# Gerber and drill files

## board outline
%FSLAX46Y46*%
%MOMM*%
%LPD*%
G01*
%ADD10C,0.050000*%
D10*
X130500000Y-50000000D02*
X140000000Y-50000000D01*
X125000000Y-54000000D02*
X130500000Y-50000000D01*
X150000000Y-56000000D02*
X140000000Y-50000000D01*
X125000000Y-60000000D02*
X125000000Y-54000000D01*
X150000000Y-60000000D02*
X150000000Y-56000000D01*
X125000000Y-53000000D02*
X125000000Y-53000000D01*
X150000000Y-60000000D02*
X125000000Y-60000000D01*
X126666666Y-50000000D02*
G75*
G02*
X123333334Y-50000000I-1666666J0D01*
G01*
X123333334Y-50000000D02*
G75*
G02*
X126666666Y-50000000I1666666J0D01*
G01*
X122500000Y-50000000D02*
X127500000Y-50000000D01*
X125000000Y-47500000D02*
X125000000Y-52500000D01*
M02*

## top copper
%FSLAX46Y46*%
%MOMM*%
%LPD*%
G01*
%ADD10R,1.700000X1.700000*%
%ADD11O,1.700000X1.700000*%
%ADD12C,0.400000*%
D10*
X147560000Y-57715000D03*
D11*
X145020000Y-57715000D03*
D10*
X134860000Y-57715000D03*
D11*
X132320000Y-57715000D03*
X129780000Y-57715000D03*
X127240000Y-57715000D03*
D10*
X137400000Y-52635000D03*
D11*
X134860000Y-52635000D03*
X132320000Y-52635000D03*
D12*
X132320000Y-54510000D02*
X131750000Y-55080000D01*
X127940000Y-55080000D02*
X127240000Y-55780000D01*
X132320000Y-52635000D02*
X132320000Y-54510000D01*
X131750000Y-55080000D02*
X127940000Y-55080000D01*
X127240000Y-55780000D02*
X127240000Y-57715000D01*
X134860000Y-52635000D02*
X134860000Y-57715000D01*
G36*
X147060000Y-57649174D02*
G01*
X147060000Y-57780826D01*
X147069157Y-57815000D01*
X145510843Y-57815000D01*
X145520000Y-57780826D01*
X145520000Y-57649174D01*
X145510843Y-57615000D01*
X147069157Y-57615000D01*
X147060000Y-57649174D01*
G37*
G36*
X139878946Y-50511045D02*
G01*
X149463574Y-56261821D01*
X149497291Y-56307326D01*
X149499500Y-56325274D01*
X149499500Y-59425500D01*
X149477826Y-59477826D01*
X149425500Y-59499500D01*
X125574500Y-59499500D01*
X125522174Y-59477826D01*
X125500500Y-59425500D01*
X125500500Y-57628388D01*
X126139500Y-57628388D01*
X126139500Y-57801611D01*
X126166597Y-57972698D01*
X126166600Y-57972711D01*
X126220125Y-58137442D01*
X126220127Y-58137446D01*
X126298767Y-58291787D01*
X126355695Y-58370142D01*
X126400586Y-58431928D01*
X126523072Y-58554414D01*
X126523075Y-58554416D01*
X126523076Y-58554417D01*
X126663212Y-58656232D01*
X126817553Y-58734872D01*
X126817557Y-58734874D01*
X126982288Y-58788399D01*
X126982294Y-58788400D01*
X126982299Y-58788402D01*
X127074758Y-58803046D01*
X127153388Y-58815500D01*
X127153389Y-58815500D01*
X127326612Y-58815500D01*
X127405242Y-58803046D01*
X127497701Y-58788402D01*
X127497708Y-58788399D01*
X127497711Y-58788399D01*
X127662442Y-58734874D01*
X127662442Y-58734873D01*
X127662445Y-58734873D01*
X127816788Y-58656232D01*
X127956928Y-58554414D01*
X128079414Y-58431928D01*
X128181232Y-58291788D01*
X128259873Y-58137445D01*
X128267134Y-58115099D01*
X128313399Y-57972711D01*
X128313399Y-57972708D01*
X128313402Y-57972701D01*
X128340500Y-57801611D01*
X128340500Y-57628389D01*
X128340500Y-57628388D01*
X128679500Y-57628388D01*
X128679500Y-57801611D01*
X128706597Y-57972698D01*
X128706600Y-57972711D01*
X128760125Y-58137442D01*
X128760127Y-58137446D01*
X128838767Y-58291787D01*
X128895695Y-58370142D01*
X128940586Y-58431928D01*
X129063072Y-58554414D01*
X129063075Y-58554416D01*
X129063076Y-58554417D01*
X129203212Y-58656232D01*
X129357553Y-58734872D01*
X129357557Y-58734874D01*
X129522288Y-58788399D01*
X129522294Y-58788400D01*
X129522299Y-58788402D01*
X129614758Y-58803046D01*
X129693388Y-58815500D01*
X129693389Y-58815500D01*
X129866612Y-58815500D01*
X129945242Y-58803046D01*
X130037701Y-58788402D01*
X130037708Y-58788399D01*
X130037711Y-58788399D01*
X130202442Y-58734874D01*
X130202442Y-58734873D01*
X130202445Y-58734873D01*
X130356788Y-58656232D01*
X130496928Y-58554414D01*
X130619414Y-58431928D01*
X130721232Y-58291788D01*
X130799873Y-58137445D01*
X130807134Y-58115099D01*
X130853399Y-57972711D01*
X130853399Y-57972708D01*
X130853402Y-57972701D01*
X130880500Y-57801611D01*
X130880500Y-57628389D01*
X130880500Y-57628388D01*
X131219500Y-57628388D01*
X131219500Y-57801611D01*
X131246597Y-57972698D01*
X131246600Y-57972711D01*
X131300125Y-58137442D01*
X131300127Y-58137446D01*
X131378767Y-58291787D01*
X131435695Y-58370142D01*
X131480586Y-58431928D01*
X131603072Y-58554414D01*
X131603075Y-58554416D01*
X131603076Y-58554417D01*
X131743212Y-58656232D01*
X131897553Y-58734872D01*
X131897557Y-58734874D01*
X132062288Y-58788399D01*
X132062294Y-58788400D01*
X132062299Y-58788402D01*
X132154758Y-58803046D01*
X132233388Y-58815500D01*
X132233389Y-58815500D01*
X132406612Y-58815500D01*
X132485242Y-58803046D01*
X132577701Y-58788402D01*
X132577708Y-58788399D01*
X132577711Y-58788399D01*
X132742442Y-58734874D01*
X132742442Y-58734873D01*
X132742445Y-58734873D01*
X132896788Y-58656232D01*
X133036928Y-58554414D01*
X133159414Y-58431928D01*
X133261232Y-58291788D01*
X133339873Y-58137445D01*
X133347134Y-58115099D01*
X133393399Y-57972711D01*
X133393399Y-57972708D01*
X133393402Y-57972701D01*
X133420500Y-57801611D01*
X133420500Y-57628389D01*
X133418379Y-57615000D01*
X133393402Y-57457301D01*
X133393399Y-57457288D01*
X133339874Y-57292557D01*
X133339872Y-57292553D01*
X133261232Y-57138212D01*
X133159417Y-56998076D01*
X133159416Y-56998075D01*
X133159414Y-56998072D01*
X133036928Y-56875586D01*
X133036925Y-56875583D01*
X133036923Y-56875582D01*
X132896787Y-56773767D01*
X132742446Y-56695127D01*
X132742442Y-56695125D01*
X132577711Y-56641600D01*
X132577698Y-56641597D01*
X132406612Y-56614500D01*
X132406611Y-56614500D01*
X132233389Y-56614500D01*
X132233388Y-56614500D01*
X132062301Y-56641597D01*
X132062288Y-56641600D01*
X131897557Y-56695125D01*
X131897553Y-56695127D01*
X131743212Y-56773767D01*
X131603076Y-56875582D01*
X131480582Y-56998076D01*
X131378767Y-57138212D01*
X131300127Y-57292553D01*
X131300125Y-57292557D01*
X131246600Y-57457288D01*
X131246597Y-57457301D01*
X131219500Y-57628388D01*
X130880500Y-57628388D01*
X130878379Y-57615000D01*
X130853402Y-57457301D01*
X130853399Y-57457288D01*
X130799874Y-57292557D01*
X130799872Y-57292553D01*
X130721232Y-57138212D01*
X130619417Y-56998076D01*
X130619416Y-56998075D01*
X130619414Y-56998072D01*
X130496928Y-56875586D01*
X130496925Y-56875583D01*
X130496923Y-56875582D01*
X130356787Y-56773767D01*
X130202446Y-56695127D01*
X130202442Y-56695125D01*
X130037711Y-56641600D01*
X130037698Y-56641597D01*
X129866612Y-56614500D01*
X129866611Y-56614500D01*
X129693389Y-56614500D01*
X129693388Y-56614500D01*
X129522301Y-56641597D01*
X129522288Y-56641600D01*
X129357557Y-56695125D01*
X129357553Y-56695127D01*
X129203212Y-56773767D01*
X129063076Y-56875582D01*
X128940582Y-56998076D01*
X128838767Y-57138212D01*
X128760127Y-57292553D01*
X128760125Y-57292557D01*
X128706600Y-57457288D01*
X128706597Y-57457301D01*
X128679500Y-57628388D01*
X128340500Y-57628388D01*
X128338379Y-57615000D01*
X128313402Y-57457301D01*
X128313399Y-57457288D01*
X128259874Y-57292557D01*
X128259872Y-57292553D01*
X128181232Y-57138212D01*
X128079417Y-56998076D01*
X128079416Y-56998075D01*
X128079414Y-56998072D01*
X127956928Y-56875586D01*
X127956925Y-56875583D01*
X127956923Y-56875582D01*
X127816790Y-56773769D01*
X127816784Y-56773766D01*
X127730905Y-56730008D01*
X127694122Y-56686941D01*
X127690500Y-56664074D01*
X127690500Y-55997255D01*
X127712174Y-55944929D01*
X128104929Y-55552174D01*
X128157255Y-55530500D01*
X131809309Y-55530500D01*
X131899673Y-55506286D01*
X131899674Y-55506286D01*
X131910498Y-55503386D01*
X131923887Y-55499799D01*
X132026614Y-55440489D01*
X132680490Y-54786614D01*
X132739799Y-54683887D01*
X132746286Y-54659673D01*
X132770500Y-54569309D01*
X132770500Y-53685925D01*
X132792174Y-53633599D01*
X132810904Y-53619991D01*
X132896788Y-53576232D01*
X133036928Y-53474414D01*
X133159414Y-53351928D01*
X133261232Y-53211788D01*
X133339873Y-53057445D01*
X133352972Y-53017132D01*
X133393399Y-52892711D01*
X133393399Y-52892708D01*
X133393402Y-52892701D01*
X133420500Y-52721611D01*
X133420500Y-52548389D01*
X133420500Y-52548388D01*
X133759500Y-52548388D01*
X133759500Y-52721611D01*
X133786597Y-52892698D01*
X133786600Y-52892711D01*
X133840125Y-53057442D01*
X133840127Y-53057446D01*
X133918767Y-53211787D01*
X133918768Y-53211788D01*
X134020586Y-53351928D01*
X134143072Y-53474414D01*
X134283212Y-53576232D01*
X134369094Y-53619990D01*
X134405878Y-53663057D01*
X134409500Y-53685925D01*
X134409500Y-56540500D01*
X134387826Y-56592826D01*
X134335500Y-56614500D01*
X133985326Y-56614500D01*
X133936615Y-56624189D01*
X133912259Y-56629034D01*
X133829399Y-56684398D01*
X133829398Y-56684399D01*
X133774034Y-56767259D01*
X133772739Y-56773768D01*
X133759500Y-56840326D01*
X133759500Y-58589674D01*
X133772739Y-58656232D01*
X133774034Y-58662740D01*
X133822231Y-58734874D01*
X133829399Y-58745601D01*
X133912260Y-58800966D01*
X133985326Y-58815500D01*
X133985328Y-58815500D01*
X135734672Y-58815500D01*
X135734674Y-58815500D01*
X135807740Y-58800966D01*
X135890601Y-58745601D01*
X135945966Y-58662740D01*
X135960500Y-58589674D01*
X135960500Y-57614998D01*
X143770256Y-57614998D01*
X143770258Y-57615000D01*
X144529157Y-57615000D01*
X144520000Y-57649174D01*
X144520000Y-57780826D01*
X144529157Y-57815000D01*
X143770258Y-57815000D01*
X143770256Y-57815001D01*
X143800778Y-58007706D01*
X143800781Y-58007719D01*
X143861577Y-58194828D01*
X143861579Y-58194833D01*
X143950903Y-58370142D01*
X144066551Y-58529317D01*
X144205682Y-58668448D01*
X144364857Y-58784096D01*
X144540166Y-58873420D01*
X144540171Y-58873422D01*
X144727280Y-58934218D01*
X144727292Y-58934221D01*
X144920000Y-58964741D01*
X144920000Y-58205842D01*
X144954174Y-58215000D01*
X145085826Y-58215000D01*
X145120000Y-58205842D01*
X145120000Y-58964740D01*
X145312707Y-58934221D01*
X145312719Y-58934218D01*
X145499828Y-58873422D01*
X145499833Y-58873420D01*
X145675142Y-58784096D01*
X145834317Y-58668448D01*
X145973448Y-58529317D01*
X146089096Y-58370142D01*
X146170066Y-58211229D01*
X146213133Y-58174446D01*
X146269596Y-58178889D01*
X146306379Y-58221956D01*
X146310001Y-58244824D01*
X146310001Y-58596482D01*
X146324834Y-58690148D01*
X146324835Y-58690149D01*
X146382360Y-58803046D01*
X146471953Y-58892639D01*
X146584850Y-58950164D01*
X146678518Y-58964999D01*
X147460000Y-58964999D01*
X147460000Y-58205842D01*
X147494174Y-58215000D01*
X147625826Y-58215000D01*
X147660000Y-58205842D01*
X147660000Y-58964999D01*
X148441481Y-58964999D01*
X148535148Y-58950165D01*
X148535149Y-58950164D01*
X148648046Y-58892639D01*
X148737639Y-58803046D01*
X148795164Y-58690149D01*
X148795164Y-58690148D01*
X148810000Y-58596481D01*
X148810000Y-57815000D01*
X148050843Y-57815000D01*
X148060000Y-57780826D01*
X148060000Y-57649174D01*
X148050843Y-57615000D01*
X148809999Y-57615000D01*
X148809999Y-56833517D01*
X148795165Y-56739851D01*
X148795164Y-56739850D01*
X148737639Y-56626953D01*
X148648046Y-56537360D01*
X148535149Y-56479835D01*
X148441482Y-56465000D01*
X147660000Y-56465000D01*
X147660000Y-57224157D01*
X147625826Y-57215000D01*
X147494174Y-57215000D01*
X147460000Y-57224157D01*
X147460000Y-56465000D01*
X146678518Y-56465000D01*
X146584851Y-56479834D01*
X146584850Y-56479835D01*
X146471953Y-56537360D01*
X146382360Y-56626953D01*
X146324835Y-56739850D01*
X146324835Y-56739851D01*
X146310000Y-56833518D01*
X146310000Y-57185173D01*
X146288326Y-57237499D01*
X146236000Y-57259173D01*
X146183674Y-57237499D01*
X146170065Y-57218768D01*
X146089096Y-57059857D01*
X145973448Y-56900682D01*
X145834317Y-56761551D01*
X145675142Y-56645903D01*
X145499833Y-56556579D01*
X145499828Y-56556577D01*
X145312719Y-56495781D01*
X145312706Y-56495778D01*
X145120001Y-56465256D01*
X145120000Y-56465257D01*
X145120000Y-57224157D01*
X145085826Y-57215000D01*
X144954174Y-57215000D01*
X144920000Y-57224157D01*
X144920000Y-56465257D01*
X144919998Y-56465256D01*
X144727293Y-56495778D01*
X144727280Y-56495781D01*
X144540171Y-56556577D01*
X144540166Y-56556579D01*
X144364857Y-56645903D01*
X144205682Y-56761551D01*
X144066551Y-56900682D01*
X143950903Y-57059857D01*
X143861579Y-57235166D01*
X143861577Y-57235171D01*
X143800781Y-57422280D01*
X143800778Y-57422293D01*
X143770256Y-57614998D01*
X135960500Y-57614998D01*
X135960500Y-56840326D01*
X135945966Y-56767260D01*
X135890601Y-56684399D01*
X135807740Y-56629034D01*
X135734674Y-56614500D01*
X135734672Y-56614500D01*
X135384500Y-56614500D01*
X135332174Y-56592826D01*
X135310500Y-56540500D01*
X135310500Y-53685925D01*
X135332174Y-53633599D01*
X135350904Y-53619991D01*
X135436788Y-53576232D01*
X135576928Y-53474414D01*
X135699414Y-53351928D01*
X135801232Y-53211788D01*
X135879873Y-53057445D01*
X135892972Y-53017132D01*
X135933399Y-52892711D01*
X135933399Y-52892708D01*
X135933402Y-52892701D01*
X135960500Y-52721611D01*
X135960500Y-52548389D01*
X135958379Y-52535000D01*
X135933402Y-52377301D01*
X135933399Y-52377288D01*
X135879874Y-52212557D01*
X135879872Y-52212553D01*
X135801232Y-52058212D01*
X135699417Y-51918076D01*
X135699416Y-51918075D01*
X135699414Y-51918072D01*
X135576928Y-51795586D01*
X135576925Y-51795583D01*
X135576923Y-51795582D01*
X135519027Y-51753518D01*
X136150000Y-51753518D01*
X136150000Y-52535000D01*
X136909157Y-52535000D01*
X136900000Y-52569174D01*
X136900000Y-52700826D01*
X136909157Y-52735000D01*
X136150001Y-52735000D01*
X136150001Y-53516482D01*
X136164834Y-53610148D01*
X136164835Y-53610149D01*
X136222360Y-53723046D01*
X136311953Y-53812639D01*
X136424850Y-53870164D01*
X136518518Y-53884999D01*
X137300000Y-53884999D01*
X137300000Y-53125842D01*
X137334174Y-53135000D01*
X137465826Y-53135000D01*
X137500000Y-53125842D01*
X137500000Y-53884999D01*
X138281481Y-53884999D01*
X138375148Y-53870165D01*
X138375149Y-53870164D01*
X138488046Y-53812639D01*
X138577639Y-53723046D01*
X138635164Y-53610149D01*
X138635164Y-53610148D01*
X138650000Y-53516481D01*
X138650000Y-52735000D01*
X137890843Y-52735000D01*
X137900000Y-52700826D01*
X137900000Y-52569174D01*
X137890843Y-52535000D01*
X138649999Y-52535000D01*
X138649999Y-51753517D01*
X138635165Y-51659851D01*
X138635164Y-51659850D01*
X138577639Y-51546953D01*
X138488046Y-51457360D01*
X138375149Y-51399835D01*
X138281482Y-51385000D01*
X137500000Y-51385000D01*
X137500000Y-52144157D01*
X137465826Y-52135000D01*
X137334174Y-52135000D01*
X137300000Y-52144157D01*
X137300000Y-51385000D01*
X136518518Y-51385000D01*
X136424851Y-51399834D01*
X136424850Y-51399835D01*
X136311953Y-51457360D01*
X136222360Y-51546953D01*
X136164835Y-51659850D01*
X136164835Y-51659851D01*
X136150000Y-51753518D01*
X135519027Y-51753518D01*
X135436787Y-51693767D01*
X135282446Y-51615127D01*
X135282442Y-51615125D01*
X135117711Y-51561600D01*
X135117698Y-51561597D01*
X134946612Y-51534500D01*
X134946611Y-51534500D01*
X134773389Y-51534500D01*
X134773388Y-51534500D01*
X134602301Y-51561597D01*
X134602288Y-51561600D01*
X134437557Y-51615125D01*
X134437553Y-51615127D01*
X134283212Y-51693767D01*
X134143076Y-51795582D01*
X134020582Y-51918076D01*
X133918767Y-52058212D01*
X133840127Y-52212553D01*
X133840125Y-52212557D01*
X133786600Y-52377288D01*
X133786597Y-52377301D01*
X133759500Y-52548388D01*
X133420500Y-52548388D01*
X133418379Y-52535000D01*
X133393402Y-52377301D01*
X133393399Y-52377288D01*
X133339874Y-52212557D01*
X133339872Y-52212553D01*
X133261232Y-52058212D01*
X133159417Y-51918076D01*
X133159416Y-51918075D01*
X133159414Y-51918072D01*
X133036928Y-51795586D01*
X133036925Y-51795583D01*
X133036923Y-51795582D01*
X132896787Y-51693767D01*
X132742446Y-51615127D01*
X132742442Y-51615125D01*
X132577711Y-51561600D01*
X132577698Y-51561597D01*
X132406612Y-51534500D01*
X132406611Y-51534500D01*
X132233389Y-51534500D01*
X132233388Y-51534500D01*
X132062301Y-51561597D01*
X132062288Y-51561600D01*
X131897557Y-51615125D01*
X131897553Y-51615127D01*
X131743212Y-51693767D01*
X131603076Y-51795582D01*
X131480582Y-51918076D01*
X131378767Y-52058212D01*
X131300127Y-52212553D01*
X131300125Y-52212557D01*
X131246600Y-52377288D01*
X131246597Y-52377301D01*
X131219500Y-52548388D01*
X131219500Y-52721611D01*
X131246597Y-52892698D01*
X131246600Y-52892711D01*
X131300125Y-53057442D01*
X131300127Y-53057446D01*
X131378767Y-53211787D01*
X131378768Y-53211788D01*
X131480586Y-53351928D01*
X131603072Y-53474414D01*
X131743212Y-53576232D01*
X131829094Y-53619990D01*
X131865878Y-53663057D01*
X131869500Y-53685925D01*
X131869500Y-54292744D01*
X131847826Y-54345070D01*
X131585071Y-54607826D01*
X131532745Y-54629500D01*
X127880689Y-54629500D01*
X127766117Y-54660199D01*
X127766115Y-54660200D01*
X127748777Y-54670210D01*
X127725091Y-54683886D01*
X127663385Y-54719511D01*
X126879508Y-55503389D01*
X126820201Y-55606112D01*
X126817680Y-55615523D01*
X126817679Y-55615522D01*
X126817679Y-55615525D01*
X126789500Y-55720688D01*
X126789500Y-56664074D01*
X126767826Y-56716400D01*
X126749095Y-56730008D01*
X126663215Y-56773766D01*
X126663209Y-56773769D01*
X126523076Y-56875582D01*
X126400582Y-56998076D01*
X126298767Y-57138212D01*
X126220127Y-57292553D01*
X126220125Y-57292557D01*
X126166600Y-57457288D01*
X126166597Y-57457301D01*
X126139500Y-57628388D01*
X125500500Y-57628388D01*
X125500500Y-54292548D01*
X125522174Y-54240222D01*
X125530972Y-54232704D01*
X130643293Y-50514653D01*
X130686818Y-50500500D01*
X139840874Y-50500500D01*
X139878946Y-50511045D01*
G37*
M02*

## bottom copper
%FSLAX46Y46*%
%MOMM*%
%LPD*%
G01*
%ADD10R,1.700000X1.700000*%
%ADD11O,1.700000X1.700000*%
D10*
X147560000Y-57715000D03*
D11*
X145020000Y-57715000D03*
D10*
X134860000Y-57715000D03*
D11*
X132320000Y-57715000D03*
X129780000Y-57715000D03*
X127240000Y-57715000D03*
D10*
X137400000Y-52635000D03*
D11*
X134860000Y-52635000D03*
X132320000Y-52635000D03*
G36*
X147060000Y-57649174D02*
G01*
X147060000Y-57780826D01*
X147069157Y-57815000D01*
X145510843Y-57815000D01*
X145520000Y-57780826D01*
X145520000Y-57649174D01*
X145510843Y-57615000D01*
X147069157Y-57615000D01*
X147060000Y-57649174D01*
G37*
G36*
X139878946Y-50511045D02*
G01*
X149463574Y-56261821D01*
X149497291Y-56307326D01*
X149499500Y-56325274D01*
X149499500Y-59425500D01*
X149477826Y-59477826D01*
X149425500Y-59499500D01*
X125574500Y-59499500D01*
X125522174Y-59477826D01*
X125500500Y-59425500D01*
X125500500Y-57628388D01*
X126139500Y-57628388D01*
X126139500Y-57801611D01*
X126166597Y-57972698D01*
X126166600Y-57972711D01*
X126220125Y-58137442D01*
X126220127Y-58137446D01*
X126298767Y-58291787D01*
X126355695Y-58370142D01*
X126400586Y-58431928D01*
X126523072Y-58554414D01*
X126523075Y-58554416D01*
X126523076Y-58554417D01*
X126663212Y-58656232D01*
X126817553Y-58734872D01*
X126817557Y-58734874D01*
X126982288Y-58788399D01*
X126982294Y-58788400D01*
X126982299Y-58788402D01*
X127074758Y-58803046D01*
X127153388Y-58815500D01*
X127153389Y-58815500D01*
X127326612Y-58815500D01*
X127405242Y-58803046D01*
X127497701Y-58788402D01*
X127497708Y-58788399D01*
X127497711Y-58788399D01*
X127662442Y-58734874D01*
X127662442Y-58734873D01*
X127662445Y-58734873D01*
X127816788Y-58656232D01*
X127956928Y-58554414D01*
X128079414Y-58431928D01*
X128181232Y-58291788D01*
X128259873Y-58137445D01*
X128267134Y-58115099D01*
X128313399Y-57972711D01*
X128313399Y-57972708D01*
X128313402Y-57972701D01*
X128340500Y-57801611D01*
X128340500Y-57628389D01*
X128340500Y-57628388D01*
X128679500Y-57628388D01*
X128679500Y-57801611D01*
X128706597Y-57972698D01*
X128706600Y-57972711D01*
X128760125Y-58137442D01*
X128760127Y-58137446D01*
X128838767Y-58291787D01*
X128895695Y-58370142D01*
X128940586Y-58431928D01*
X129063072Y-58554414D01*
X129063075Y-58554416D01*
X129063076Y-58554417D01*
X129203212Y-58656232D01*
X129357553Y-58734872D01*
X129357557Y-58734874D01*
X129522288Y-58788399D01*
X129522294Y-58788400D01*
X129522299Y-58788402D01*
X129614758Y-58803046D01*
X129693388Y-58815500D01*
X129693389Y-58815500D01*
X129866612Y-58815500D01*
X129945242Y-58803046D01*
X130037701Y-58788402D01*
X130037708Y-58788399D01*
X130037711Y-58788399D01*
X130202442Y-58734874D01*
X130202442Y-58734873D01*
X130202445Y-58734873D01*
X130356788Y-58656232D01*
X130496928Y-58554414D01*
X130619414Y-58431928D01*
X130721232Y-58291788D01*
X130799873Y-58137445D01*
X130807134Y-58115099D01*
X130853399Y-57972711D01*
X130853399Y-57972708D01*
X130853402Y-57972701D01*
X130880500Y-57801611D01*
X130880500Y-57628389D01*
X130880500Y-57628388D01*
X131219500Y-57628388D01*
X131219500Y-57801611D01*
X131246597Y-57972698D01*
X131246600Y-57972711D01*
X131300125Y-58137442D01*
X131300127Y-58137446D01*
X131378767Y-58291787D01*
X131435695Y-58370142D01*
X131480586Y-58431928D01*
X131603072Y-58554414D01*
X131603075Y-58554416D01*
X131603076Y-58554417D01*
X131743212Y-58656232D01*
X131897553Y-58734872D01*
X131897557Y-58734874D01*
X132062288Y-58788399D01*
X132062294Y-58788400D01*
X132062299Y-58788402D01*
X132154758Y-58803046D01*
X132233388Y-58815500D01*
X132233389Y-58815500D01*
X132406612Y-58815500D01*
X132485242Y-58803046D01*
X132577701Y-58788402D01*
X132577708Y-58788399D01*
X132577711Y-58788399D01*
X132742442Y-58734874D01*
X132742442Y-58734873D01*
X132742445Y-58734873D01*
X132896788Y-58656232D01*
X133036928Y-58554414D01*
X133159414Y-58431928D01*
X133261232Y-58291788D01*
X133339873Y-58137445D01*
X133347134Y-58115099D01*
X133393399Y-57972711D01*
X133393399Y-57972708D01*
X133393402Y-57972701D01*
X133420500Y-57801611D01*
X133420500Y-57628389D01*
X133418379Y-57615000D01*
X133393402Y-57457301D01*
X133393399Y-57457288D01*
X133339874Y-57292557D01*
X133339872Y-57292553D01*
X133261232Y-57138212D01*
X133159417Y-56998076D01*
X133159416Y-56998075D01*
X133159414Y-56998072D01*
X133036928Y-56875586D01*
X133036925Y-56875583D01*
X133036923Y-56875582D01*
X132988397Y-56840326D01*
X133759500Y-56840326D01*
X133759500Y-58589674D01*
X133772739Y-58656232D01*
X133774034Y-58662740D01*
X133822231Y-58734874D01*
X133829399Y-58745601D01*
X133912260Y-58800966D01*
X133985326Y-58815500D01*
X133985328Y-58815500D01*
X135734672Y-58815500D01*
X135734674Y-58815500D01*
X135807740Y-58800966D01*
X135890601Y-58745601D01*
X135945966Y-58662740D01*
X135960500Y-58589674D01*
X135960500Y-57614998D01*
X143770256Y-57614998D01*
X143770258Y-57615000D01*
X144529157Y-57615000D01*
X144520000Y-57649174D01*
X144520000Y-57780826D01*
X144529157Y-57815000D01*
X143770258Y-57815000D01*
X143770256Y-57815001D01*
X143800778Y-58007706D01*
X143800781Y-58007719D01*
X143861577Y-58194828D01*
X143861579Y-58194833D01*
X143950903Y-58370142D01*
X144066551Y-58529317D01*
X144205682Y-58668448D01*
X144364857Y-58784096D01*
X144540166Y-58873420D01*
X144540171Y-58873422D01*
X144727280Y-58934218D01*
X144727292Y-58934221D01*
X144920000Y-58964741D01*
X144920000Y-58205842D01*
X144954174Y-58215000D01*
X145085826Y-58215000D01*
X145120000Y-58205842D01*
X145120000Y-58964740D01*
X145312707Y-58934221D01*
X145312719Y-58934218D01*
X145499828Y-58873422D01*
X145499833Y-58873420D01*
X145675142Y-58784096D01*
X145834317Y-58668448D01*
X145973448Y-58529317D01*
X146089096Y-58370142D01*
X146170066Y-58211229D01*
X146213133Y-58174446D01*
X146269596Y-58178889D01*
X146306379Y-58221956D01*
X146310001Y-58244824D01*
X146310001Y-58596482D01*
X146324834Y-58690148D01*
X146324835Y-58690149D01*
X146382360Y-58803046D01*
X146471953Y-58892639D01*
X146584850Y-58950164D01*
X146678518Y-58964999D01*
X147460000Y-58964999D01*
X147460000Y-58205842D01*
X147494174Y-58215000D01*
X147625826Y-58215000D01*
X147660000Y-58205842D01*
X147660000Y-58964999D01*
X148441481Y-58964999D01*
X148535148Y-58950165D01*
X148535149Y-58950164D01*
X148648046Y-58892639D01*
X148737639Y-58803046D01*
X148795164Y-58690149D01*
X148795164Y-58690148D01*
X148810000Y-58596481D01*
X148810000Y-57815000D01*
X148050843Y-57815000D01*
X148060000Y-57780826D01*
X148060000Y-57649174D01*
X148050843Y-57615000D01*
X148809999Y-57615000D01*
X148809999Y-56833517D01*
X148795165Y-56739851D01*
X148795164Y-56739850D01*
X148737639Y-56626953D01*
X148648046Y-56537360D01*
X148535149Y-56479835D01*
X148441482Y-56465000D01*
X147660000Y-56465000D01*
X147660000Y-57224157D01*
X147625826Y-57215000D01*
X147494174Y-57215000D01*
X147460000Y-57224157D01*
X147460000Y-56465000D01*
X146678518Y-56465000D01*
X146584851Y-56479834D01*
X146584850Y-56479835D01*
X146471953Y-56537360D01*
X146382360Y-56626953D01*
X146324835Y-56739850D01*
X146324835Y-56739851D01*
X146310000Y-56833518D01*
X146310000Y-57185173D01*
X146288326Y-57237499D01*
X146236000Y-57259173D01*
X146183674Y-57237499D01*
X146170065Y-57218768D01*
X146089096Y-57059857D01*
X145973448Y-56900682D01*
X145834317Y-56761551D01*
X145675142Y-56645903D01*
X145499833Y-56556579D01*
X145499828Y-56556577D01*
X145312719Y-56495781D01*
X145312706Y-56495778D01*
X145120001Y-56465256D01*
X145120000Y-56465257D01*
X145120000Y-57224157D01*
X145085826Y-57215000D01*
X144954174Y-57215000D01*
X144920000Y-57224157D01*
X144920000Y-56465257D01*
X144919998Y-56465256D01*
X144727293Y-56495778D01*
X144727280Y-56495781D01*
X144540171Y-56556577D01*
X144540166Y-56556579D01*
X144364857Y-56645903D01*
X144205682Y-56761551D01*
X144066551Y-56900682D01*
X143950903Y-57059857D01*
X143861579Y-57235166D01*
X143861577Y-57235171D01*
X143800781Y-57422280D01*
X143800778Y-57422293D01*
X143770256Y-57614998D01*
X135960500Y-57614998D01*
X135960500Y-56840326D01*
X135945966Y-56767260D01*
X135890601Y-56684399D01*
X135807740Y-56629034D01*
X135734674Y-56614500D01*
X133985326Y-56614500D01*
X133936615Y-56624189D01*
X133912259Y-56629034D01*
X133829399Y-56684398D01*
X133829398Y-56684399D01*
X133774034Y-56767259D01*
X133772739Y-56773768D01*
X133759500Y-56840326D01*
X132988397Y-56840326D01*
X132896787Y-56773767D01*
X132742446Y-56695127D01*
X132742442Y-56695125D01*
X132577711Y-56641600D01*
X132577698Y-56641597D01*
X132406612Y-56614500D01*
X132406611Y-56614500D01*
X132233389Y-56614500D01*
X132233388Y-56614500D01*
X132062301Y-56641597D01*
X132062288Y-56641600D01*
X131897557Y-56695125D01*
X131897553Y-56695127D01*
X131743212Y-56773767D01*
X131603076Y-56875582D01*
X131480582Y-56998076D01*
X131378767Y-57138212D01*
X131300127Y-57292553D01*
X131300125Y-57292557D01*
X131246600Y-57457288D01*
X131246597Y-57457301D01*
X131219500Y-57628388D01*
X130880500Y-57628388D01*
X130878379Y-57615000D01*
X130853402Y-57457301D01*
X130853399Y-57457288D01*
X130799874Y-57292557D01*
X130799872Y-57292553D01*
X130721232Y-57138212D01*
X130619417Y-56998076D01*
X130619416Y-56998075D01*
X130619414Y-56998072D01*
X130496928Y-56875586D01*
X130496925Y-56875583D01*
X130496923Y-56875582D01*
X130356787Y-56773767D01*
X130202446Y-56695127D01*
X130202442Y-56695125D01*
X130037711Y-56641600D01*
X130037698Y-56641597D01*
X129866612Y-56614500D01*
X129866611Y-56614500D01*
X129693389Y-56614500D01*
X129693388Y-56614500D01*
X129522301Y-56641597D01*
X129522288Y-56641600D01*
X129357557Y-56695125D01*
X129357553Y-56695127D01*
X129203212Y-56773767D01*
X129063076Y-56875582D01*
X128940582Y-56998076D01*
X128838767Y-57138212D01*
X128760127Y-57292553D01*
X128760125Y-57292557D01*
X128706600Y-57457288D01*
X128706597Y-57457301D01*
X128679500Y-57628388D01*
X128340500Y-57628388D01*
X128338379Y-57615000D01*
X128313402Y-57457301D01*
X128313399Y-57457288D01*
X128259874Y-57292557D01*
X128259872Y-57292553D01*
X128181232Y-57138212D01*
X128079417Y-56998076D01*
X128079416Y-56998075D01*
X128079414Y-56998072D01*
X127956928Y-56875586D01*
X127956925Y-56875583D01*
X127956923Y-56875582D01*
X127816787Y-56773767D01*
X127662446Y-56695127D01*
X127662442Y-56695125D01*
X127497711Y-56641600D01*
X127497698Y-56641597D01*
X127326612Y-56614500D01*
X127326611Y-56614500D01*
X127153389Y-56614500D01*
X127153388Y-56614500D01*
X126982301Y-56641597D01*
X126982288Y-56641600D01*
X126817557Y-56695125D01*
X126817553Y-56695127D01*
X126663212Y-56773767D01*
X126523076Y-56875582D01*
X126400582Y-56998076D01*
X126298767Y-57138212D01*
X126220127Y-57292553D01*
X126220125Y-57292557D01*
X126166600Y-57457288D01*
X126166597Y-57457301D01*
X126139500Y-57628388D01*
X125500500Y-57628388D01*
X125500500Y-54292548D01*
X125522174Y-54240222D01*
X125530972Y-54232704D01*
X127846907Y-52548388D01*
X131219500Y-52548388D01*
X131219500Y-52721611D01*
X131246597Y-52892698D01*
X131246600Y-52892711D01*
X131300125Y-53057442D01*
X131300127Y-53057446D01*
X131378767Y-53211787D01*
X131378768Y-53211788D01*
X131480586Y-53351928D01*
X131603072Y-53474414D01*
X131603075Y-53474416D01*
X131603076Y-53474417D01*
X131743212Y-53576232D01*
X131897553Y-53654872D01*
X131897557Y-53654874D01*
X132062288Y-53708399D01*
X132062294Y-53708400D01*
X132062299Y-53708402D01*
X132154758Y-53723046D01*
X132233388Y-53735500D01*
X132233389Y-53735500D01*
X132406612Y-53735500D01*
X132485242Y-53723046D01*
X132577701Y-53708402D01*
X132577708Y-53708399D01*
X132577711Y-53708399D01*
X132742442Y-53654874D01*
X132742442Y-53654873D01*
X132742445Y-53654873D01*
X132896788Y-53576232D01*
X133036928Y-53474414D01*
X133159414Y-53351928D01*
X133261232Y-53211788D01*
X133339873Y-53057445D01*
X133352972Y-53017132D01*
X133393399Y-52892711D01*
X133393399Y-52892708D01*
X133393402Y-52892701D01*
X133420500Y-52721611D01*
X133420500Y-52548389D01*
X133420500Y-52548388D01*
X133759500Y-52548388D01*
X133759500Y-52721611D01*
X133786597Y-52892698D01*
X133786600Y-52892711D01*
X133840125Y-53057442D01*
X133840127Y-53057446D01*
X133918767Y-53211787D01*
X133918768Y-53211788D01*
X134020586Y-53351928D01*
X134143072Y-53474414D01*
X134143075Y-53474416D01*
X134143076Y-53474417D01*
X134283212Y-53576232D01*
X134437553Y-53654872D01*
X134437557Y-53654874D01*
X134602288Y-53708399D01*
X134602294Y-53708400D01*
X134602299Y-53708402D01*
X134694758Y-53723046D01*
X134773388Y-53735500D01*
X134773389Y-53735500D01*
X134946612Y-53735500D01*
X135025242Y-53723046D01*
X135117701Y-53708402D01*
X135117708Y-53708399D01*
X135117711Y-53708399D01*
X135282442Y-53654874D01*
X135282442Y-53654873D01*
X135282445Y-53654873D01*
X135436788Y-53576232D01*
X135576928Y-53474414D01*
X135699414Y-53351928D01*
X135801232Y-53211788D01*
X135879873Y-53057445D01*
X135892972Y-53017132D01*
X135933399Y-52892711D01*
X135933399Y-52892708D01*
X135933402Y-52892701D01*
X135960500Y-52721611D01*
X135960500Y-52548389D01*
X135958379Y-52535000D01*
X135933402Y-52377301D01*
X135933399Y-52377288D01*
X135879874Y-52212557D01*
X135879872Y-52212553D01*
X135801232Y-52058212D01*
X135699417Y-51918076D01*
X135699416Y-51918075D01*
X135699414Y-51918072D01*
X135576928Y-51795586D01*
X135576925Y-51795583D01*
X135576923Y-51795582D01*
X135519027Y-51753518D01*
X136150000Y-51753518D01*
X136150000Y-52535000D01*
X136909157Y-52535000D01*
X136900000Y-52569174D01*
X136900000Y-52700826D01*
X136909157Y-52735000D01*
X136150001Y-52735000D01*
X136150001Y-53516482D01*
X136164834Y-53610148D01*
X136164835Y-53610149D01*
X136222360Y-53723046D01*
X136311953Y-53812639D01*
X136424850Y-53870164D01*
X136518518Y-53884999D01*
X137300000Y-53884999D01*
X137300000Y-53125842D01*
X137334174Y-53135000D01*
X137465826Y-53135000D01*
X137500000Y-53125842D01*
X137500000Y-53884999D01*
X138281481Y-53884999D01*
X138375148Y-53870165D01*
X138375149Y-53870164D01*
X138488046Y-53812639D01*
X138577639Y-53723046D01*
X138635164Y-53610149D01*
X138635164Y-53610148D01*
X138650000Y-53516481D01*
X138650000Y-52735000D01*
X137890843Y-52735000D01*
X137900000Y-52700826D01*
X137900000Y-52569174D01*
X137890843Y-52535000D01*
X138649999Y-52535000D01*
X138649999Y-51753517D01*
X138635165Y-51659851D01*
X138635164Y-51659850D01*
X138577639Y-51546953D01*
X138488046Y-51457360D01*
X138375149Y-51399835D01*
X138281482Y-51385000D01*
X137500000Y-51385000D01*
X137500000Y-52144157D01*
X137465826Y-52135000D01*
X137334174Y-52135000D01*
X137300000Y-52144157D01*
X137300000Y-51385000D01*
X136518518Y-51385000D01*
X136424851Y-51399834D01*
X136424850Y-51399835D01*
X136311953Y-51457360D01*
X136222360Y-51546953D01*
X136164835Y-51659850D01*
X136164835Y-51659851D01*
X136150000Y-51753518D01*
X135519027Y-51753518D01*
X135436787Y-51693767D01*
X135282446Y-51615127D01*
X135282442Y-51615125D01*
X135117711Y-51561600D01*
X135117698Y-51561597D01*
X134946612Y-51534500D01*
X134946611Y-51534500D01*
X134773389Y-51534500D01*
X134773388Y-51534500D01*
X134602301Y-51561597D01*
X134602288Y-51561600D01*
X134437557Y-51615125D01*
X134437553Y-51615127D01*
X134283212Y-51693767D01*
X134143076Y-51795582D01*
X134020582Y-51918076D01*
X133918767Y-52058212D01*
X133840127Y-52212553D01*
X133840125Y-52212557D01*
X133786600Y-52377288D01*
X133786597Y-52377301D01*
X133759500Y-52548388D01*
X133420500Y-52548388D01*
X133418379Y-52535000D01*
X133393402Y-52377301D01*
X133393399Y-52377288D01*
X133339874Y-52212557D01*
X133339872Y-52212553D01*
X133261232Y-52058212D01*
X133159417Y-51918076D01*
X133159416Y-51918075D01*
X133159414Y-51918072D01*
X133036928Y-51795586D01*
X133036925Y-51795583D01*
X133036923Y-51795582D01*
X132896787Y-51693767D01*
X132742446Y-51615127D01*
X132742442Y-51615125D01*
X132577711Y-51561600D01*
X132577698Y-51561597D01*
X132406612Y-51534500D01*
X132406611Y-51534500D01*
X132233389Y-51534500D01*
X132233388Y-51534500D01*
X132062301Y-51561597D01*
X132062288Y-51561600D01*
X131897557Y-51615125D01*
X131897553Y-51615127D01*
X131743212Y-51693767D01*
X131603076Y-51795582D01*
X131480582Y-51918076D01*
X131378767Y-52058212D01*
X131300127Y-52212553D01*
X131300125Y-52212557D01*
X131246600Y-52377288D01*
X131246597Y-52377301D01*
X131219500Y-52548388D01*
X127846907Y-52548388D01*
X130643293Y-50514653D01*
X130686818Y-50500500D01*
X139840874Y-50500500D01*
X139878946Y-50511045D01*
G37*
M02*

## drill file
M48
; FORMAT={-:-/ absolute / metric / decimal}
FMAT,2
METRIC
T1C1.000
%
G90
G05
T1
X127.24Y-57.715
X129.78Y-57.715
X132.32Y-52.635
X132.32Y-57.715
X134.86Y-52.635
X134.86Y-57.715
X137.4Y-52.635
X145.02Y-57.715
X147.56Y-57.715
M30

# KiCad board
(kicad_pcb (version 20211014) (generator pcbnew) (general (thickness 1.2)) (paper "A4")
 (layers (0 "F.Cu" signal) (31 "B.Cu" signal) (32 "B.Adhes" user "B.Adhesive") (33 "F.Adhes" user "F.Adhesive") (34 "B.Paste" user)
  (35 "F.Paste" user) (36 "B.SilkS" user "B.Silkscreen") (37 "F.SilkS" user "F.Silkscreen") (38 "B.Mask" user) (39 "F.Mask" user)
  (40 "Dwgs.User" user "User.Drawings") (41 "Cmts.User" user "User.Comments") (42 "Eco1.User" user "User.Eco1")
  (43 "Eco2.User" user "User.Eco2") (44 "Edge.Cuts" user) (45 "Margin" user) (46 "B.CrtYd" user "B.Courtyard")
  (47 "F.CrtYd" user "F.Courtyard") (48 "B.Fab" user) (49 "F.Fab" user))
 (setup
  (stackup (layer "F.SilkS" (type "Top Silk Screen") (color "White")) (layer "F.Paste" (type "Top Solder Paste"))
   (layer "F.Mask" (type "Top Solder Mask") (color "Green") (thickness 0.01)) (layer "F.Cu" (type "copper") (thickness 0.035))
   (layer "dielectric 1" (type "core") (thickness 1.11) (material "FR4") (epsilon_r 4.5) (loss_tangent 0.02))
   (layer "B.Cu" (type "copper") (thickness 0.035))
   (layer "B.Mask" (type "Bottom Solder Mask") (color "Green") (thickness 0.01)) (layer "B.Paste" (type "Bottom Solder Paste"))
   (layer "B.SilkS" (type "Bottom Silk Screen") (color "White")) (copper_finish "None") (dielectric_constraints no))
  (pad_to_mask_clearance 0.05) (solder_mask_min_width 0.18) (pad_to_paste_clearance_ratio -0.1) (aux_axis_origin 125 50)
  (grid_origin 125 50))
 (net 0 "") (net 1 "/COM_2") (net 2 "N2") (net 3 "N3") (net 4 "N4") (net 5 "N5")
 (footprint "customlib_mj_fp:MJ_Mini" (layer "F.Cu") (at 139.94 57.08)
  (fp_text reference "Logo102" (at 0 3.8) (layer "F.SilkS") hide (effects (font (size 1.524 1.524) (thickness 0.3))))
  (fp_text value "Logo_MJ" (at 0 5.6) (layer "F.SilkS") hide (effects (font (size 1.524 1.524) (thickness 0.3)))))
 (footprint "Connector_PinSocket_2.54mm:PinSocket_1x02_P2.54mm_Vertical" (layer "B.Cu") (at 147.56 57.715 90)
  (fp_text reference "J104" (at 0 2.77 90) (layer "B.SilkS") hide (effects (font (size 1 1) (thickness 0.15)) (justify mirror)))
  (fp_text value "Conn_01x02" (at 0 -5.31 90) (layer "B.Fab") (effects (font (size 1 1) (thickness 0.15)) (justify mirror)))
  (pad "1" thru_hole rect locked (at 0 0 90) (size 1.7 1.7) (drill 1) (layers *.Cu *.Mask) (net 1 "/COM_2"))
  (pad "2" thru_hole oval locked (at 0 -2.54 90) (size 1.7 1.7) (drill 1) (layers *.Cu *.Mask) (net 1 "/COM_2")))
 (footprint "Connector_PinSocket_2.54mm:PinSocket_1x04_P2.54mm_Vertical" (layer "B.Cu") (at 134.86 57.715 90)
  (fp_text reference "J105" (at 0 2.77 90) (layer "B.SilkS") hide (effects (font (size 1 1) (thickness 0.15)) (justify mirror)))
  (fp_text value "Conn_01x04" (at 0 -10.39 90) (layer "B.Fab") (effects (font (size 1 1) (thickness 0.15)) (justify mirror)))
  (pad "1" thru_hole rect locked (at 0 0 90) (size 1.7 1.7) (drill 1) (layers *.Cu *.Mask) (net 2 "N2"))
  (pad "2" thru_hole oval locked (at 0 -2.54 90) (size 1.7 1.7) (drill 1) (layers *.Cu *.Mask) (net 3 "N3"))
  (pad "3" thru_hole oval locked (at 0 -5.08 90) (size 1.7 1.7) (drill 1) (layers *.Cu *.Mask) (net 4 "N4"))
  (pad "4" thru_hole oval locked (at 0 -7.62 90) (size 1.7 1.7) (drill 1) (layers *.Cu *.Mask) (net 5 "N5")))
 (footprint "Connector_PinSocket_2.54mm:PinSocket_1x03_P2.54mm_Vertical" (layer "B.Cu") (at 137.4 52.635 90)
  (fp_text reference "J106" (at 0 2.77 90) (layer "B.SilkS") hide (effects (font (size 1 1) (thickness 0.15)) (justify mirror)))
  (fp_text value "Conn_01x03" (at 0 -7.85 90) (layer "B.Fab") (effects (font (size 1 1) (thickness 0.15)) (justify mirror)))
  (pad "1" thru_hole rect locked (at 0 0 90) (size 1.7 1.7) (drill 1) (layers *.Cu *.Mask) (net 1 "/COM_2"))
  (pad "2" thru_hole oval locked (at 0 -2.54 90) (size 1.7 1.7) (drill 1) (layers *.Cu *.Mask) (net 2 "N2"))
  (pad "3" thru_hole oval locked (at 0 -5.08 90) (size 1.7 1.7) (drill 1) (layers *.Cu *.Mask) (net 5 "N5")))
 (gr_line (start 130.5 50) (end 140 50) (layer "Edge.Cuts") (width 0.05))
 (gr_line (start 125 54) (end 130.5 50) (layer "Edge.Cuts") (width 0.05))
 (gr_line (start 150 56) (end 140 50) (layer "Edge.Cuts") (width 0.05))
 (gr_line (start 125 60) (end 125 54) (layer "Edge.Cuts") (width 0.05))
 (gr_line (start 150 60) (end 150 56) (layer "Edge.Cuts") (width 0.05))
 (gr_line (start 125 53) (end 125 53) (layer "Edge.Cuts") (width 0.05))
 (gr_line (start 150 60) (end 125 60) (layer "Edge.Cuts") (width 0.05))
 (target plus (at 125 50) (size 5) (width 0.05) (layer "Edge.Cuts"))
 (segment (start 132.32 54.51) (end 131.75 55.08) (width 0.4) (layer "F.Cu") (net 5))
 (segment (start 127.94 55.08) (end 127.24 55.78) (width 0.4) (layer "F.Cu") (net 5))
 (segment (start 132.32 52.635) (end 132.32 54.51) (width 0.4) (layer "F.Cu") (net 5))
 (segment (start 131.75 55.08) (end 127.94 55.08) (width 0.4) (layer "F.Cu") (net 5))
 (segment (start 127.24 55.78) (end 127.24 57.715) (width 0.4) (layer "F.Cu") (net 5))
 (segment (start 134.86 52.635) (end 134.86 57.715) (width 0.4) (layer "F.Cu") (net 2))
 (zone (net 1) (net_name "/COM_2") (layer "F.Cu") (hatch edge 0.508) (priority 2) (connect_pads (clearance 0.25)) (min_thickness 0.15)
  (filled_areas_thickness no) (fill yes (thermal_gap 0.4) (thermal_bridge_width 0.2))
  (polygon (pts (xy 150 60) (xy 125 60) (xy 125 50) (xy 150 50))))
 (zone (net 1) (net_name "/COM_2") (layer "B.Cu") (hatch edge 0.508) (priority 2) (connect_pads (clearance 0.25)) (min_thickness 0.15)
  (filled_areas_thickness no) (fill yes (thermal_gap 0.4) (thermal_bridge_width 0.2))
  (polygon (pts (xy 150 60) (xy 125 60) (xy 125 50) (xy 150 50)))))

